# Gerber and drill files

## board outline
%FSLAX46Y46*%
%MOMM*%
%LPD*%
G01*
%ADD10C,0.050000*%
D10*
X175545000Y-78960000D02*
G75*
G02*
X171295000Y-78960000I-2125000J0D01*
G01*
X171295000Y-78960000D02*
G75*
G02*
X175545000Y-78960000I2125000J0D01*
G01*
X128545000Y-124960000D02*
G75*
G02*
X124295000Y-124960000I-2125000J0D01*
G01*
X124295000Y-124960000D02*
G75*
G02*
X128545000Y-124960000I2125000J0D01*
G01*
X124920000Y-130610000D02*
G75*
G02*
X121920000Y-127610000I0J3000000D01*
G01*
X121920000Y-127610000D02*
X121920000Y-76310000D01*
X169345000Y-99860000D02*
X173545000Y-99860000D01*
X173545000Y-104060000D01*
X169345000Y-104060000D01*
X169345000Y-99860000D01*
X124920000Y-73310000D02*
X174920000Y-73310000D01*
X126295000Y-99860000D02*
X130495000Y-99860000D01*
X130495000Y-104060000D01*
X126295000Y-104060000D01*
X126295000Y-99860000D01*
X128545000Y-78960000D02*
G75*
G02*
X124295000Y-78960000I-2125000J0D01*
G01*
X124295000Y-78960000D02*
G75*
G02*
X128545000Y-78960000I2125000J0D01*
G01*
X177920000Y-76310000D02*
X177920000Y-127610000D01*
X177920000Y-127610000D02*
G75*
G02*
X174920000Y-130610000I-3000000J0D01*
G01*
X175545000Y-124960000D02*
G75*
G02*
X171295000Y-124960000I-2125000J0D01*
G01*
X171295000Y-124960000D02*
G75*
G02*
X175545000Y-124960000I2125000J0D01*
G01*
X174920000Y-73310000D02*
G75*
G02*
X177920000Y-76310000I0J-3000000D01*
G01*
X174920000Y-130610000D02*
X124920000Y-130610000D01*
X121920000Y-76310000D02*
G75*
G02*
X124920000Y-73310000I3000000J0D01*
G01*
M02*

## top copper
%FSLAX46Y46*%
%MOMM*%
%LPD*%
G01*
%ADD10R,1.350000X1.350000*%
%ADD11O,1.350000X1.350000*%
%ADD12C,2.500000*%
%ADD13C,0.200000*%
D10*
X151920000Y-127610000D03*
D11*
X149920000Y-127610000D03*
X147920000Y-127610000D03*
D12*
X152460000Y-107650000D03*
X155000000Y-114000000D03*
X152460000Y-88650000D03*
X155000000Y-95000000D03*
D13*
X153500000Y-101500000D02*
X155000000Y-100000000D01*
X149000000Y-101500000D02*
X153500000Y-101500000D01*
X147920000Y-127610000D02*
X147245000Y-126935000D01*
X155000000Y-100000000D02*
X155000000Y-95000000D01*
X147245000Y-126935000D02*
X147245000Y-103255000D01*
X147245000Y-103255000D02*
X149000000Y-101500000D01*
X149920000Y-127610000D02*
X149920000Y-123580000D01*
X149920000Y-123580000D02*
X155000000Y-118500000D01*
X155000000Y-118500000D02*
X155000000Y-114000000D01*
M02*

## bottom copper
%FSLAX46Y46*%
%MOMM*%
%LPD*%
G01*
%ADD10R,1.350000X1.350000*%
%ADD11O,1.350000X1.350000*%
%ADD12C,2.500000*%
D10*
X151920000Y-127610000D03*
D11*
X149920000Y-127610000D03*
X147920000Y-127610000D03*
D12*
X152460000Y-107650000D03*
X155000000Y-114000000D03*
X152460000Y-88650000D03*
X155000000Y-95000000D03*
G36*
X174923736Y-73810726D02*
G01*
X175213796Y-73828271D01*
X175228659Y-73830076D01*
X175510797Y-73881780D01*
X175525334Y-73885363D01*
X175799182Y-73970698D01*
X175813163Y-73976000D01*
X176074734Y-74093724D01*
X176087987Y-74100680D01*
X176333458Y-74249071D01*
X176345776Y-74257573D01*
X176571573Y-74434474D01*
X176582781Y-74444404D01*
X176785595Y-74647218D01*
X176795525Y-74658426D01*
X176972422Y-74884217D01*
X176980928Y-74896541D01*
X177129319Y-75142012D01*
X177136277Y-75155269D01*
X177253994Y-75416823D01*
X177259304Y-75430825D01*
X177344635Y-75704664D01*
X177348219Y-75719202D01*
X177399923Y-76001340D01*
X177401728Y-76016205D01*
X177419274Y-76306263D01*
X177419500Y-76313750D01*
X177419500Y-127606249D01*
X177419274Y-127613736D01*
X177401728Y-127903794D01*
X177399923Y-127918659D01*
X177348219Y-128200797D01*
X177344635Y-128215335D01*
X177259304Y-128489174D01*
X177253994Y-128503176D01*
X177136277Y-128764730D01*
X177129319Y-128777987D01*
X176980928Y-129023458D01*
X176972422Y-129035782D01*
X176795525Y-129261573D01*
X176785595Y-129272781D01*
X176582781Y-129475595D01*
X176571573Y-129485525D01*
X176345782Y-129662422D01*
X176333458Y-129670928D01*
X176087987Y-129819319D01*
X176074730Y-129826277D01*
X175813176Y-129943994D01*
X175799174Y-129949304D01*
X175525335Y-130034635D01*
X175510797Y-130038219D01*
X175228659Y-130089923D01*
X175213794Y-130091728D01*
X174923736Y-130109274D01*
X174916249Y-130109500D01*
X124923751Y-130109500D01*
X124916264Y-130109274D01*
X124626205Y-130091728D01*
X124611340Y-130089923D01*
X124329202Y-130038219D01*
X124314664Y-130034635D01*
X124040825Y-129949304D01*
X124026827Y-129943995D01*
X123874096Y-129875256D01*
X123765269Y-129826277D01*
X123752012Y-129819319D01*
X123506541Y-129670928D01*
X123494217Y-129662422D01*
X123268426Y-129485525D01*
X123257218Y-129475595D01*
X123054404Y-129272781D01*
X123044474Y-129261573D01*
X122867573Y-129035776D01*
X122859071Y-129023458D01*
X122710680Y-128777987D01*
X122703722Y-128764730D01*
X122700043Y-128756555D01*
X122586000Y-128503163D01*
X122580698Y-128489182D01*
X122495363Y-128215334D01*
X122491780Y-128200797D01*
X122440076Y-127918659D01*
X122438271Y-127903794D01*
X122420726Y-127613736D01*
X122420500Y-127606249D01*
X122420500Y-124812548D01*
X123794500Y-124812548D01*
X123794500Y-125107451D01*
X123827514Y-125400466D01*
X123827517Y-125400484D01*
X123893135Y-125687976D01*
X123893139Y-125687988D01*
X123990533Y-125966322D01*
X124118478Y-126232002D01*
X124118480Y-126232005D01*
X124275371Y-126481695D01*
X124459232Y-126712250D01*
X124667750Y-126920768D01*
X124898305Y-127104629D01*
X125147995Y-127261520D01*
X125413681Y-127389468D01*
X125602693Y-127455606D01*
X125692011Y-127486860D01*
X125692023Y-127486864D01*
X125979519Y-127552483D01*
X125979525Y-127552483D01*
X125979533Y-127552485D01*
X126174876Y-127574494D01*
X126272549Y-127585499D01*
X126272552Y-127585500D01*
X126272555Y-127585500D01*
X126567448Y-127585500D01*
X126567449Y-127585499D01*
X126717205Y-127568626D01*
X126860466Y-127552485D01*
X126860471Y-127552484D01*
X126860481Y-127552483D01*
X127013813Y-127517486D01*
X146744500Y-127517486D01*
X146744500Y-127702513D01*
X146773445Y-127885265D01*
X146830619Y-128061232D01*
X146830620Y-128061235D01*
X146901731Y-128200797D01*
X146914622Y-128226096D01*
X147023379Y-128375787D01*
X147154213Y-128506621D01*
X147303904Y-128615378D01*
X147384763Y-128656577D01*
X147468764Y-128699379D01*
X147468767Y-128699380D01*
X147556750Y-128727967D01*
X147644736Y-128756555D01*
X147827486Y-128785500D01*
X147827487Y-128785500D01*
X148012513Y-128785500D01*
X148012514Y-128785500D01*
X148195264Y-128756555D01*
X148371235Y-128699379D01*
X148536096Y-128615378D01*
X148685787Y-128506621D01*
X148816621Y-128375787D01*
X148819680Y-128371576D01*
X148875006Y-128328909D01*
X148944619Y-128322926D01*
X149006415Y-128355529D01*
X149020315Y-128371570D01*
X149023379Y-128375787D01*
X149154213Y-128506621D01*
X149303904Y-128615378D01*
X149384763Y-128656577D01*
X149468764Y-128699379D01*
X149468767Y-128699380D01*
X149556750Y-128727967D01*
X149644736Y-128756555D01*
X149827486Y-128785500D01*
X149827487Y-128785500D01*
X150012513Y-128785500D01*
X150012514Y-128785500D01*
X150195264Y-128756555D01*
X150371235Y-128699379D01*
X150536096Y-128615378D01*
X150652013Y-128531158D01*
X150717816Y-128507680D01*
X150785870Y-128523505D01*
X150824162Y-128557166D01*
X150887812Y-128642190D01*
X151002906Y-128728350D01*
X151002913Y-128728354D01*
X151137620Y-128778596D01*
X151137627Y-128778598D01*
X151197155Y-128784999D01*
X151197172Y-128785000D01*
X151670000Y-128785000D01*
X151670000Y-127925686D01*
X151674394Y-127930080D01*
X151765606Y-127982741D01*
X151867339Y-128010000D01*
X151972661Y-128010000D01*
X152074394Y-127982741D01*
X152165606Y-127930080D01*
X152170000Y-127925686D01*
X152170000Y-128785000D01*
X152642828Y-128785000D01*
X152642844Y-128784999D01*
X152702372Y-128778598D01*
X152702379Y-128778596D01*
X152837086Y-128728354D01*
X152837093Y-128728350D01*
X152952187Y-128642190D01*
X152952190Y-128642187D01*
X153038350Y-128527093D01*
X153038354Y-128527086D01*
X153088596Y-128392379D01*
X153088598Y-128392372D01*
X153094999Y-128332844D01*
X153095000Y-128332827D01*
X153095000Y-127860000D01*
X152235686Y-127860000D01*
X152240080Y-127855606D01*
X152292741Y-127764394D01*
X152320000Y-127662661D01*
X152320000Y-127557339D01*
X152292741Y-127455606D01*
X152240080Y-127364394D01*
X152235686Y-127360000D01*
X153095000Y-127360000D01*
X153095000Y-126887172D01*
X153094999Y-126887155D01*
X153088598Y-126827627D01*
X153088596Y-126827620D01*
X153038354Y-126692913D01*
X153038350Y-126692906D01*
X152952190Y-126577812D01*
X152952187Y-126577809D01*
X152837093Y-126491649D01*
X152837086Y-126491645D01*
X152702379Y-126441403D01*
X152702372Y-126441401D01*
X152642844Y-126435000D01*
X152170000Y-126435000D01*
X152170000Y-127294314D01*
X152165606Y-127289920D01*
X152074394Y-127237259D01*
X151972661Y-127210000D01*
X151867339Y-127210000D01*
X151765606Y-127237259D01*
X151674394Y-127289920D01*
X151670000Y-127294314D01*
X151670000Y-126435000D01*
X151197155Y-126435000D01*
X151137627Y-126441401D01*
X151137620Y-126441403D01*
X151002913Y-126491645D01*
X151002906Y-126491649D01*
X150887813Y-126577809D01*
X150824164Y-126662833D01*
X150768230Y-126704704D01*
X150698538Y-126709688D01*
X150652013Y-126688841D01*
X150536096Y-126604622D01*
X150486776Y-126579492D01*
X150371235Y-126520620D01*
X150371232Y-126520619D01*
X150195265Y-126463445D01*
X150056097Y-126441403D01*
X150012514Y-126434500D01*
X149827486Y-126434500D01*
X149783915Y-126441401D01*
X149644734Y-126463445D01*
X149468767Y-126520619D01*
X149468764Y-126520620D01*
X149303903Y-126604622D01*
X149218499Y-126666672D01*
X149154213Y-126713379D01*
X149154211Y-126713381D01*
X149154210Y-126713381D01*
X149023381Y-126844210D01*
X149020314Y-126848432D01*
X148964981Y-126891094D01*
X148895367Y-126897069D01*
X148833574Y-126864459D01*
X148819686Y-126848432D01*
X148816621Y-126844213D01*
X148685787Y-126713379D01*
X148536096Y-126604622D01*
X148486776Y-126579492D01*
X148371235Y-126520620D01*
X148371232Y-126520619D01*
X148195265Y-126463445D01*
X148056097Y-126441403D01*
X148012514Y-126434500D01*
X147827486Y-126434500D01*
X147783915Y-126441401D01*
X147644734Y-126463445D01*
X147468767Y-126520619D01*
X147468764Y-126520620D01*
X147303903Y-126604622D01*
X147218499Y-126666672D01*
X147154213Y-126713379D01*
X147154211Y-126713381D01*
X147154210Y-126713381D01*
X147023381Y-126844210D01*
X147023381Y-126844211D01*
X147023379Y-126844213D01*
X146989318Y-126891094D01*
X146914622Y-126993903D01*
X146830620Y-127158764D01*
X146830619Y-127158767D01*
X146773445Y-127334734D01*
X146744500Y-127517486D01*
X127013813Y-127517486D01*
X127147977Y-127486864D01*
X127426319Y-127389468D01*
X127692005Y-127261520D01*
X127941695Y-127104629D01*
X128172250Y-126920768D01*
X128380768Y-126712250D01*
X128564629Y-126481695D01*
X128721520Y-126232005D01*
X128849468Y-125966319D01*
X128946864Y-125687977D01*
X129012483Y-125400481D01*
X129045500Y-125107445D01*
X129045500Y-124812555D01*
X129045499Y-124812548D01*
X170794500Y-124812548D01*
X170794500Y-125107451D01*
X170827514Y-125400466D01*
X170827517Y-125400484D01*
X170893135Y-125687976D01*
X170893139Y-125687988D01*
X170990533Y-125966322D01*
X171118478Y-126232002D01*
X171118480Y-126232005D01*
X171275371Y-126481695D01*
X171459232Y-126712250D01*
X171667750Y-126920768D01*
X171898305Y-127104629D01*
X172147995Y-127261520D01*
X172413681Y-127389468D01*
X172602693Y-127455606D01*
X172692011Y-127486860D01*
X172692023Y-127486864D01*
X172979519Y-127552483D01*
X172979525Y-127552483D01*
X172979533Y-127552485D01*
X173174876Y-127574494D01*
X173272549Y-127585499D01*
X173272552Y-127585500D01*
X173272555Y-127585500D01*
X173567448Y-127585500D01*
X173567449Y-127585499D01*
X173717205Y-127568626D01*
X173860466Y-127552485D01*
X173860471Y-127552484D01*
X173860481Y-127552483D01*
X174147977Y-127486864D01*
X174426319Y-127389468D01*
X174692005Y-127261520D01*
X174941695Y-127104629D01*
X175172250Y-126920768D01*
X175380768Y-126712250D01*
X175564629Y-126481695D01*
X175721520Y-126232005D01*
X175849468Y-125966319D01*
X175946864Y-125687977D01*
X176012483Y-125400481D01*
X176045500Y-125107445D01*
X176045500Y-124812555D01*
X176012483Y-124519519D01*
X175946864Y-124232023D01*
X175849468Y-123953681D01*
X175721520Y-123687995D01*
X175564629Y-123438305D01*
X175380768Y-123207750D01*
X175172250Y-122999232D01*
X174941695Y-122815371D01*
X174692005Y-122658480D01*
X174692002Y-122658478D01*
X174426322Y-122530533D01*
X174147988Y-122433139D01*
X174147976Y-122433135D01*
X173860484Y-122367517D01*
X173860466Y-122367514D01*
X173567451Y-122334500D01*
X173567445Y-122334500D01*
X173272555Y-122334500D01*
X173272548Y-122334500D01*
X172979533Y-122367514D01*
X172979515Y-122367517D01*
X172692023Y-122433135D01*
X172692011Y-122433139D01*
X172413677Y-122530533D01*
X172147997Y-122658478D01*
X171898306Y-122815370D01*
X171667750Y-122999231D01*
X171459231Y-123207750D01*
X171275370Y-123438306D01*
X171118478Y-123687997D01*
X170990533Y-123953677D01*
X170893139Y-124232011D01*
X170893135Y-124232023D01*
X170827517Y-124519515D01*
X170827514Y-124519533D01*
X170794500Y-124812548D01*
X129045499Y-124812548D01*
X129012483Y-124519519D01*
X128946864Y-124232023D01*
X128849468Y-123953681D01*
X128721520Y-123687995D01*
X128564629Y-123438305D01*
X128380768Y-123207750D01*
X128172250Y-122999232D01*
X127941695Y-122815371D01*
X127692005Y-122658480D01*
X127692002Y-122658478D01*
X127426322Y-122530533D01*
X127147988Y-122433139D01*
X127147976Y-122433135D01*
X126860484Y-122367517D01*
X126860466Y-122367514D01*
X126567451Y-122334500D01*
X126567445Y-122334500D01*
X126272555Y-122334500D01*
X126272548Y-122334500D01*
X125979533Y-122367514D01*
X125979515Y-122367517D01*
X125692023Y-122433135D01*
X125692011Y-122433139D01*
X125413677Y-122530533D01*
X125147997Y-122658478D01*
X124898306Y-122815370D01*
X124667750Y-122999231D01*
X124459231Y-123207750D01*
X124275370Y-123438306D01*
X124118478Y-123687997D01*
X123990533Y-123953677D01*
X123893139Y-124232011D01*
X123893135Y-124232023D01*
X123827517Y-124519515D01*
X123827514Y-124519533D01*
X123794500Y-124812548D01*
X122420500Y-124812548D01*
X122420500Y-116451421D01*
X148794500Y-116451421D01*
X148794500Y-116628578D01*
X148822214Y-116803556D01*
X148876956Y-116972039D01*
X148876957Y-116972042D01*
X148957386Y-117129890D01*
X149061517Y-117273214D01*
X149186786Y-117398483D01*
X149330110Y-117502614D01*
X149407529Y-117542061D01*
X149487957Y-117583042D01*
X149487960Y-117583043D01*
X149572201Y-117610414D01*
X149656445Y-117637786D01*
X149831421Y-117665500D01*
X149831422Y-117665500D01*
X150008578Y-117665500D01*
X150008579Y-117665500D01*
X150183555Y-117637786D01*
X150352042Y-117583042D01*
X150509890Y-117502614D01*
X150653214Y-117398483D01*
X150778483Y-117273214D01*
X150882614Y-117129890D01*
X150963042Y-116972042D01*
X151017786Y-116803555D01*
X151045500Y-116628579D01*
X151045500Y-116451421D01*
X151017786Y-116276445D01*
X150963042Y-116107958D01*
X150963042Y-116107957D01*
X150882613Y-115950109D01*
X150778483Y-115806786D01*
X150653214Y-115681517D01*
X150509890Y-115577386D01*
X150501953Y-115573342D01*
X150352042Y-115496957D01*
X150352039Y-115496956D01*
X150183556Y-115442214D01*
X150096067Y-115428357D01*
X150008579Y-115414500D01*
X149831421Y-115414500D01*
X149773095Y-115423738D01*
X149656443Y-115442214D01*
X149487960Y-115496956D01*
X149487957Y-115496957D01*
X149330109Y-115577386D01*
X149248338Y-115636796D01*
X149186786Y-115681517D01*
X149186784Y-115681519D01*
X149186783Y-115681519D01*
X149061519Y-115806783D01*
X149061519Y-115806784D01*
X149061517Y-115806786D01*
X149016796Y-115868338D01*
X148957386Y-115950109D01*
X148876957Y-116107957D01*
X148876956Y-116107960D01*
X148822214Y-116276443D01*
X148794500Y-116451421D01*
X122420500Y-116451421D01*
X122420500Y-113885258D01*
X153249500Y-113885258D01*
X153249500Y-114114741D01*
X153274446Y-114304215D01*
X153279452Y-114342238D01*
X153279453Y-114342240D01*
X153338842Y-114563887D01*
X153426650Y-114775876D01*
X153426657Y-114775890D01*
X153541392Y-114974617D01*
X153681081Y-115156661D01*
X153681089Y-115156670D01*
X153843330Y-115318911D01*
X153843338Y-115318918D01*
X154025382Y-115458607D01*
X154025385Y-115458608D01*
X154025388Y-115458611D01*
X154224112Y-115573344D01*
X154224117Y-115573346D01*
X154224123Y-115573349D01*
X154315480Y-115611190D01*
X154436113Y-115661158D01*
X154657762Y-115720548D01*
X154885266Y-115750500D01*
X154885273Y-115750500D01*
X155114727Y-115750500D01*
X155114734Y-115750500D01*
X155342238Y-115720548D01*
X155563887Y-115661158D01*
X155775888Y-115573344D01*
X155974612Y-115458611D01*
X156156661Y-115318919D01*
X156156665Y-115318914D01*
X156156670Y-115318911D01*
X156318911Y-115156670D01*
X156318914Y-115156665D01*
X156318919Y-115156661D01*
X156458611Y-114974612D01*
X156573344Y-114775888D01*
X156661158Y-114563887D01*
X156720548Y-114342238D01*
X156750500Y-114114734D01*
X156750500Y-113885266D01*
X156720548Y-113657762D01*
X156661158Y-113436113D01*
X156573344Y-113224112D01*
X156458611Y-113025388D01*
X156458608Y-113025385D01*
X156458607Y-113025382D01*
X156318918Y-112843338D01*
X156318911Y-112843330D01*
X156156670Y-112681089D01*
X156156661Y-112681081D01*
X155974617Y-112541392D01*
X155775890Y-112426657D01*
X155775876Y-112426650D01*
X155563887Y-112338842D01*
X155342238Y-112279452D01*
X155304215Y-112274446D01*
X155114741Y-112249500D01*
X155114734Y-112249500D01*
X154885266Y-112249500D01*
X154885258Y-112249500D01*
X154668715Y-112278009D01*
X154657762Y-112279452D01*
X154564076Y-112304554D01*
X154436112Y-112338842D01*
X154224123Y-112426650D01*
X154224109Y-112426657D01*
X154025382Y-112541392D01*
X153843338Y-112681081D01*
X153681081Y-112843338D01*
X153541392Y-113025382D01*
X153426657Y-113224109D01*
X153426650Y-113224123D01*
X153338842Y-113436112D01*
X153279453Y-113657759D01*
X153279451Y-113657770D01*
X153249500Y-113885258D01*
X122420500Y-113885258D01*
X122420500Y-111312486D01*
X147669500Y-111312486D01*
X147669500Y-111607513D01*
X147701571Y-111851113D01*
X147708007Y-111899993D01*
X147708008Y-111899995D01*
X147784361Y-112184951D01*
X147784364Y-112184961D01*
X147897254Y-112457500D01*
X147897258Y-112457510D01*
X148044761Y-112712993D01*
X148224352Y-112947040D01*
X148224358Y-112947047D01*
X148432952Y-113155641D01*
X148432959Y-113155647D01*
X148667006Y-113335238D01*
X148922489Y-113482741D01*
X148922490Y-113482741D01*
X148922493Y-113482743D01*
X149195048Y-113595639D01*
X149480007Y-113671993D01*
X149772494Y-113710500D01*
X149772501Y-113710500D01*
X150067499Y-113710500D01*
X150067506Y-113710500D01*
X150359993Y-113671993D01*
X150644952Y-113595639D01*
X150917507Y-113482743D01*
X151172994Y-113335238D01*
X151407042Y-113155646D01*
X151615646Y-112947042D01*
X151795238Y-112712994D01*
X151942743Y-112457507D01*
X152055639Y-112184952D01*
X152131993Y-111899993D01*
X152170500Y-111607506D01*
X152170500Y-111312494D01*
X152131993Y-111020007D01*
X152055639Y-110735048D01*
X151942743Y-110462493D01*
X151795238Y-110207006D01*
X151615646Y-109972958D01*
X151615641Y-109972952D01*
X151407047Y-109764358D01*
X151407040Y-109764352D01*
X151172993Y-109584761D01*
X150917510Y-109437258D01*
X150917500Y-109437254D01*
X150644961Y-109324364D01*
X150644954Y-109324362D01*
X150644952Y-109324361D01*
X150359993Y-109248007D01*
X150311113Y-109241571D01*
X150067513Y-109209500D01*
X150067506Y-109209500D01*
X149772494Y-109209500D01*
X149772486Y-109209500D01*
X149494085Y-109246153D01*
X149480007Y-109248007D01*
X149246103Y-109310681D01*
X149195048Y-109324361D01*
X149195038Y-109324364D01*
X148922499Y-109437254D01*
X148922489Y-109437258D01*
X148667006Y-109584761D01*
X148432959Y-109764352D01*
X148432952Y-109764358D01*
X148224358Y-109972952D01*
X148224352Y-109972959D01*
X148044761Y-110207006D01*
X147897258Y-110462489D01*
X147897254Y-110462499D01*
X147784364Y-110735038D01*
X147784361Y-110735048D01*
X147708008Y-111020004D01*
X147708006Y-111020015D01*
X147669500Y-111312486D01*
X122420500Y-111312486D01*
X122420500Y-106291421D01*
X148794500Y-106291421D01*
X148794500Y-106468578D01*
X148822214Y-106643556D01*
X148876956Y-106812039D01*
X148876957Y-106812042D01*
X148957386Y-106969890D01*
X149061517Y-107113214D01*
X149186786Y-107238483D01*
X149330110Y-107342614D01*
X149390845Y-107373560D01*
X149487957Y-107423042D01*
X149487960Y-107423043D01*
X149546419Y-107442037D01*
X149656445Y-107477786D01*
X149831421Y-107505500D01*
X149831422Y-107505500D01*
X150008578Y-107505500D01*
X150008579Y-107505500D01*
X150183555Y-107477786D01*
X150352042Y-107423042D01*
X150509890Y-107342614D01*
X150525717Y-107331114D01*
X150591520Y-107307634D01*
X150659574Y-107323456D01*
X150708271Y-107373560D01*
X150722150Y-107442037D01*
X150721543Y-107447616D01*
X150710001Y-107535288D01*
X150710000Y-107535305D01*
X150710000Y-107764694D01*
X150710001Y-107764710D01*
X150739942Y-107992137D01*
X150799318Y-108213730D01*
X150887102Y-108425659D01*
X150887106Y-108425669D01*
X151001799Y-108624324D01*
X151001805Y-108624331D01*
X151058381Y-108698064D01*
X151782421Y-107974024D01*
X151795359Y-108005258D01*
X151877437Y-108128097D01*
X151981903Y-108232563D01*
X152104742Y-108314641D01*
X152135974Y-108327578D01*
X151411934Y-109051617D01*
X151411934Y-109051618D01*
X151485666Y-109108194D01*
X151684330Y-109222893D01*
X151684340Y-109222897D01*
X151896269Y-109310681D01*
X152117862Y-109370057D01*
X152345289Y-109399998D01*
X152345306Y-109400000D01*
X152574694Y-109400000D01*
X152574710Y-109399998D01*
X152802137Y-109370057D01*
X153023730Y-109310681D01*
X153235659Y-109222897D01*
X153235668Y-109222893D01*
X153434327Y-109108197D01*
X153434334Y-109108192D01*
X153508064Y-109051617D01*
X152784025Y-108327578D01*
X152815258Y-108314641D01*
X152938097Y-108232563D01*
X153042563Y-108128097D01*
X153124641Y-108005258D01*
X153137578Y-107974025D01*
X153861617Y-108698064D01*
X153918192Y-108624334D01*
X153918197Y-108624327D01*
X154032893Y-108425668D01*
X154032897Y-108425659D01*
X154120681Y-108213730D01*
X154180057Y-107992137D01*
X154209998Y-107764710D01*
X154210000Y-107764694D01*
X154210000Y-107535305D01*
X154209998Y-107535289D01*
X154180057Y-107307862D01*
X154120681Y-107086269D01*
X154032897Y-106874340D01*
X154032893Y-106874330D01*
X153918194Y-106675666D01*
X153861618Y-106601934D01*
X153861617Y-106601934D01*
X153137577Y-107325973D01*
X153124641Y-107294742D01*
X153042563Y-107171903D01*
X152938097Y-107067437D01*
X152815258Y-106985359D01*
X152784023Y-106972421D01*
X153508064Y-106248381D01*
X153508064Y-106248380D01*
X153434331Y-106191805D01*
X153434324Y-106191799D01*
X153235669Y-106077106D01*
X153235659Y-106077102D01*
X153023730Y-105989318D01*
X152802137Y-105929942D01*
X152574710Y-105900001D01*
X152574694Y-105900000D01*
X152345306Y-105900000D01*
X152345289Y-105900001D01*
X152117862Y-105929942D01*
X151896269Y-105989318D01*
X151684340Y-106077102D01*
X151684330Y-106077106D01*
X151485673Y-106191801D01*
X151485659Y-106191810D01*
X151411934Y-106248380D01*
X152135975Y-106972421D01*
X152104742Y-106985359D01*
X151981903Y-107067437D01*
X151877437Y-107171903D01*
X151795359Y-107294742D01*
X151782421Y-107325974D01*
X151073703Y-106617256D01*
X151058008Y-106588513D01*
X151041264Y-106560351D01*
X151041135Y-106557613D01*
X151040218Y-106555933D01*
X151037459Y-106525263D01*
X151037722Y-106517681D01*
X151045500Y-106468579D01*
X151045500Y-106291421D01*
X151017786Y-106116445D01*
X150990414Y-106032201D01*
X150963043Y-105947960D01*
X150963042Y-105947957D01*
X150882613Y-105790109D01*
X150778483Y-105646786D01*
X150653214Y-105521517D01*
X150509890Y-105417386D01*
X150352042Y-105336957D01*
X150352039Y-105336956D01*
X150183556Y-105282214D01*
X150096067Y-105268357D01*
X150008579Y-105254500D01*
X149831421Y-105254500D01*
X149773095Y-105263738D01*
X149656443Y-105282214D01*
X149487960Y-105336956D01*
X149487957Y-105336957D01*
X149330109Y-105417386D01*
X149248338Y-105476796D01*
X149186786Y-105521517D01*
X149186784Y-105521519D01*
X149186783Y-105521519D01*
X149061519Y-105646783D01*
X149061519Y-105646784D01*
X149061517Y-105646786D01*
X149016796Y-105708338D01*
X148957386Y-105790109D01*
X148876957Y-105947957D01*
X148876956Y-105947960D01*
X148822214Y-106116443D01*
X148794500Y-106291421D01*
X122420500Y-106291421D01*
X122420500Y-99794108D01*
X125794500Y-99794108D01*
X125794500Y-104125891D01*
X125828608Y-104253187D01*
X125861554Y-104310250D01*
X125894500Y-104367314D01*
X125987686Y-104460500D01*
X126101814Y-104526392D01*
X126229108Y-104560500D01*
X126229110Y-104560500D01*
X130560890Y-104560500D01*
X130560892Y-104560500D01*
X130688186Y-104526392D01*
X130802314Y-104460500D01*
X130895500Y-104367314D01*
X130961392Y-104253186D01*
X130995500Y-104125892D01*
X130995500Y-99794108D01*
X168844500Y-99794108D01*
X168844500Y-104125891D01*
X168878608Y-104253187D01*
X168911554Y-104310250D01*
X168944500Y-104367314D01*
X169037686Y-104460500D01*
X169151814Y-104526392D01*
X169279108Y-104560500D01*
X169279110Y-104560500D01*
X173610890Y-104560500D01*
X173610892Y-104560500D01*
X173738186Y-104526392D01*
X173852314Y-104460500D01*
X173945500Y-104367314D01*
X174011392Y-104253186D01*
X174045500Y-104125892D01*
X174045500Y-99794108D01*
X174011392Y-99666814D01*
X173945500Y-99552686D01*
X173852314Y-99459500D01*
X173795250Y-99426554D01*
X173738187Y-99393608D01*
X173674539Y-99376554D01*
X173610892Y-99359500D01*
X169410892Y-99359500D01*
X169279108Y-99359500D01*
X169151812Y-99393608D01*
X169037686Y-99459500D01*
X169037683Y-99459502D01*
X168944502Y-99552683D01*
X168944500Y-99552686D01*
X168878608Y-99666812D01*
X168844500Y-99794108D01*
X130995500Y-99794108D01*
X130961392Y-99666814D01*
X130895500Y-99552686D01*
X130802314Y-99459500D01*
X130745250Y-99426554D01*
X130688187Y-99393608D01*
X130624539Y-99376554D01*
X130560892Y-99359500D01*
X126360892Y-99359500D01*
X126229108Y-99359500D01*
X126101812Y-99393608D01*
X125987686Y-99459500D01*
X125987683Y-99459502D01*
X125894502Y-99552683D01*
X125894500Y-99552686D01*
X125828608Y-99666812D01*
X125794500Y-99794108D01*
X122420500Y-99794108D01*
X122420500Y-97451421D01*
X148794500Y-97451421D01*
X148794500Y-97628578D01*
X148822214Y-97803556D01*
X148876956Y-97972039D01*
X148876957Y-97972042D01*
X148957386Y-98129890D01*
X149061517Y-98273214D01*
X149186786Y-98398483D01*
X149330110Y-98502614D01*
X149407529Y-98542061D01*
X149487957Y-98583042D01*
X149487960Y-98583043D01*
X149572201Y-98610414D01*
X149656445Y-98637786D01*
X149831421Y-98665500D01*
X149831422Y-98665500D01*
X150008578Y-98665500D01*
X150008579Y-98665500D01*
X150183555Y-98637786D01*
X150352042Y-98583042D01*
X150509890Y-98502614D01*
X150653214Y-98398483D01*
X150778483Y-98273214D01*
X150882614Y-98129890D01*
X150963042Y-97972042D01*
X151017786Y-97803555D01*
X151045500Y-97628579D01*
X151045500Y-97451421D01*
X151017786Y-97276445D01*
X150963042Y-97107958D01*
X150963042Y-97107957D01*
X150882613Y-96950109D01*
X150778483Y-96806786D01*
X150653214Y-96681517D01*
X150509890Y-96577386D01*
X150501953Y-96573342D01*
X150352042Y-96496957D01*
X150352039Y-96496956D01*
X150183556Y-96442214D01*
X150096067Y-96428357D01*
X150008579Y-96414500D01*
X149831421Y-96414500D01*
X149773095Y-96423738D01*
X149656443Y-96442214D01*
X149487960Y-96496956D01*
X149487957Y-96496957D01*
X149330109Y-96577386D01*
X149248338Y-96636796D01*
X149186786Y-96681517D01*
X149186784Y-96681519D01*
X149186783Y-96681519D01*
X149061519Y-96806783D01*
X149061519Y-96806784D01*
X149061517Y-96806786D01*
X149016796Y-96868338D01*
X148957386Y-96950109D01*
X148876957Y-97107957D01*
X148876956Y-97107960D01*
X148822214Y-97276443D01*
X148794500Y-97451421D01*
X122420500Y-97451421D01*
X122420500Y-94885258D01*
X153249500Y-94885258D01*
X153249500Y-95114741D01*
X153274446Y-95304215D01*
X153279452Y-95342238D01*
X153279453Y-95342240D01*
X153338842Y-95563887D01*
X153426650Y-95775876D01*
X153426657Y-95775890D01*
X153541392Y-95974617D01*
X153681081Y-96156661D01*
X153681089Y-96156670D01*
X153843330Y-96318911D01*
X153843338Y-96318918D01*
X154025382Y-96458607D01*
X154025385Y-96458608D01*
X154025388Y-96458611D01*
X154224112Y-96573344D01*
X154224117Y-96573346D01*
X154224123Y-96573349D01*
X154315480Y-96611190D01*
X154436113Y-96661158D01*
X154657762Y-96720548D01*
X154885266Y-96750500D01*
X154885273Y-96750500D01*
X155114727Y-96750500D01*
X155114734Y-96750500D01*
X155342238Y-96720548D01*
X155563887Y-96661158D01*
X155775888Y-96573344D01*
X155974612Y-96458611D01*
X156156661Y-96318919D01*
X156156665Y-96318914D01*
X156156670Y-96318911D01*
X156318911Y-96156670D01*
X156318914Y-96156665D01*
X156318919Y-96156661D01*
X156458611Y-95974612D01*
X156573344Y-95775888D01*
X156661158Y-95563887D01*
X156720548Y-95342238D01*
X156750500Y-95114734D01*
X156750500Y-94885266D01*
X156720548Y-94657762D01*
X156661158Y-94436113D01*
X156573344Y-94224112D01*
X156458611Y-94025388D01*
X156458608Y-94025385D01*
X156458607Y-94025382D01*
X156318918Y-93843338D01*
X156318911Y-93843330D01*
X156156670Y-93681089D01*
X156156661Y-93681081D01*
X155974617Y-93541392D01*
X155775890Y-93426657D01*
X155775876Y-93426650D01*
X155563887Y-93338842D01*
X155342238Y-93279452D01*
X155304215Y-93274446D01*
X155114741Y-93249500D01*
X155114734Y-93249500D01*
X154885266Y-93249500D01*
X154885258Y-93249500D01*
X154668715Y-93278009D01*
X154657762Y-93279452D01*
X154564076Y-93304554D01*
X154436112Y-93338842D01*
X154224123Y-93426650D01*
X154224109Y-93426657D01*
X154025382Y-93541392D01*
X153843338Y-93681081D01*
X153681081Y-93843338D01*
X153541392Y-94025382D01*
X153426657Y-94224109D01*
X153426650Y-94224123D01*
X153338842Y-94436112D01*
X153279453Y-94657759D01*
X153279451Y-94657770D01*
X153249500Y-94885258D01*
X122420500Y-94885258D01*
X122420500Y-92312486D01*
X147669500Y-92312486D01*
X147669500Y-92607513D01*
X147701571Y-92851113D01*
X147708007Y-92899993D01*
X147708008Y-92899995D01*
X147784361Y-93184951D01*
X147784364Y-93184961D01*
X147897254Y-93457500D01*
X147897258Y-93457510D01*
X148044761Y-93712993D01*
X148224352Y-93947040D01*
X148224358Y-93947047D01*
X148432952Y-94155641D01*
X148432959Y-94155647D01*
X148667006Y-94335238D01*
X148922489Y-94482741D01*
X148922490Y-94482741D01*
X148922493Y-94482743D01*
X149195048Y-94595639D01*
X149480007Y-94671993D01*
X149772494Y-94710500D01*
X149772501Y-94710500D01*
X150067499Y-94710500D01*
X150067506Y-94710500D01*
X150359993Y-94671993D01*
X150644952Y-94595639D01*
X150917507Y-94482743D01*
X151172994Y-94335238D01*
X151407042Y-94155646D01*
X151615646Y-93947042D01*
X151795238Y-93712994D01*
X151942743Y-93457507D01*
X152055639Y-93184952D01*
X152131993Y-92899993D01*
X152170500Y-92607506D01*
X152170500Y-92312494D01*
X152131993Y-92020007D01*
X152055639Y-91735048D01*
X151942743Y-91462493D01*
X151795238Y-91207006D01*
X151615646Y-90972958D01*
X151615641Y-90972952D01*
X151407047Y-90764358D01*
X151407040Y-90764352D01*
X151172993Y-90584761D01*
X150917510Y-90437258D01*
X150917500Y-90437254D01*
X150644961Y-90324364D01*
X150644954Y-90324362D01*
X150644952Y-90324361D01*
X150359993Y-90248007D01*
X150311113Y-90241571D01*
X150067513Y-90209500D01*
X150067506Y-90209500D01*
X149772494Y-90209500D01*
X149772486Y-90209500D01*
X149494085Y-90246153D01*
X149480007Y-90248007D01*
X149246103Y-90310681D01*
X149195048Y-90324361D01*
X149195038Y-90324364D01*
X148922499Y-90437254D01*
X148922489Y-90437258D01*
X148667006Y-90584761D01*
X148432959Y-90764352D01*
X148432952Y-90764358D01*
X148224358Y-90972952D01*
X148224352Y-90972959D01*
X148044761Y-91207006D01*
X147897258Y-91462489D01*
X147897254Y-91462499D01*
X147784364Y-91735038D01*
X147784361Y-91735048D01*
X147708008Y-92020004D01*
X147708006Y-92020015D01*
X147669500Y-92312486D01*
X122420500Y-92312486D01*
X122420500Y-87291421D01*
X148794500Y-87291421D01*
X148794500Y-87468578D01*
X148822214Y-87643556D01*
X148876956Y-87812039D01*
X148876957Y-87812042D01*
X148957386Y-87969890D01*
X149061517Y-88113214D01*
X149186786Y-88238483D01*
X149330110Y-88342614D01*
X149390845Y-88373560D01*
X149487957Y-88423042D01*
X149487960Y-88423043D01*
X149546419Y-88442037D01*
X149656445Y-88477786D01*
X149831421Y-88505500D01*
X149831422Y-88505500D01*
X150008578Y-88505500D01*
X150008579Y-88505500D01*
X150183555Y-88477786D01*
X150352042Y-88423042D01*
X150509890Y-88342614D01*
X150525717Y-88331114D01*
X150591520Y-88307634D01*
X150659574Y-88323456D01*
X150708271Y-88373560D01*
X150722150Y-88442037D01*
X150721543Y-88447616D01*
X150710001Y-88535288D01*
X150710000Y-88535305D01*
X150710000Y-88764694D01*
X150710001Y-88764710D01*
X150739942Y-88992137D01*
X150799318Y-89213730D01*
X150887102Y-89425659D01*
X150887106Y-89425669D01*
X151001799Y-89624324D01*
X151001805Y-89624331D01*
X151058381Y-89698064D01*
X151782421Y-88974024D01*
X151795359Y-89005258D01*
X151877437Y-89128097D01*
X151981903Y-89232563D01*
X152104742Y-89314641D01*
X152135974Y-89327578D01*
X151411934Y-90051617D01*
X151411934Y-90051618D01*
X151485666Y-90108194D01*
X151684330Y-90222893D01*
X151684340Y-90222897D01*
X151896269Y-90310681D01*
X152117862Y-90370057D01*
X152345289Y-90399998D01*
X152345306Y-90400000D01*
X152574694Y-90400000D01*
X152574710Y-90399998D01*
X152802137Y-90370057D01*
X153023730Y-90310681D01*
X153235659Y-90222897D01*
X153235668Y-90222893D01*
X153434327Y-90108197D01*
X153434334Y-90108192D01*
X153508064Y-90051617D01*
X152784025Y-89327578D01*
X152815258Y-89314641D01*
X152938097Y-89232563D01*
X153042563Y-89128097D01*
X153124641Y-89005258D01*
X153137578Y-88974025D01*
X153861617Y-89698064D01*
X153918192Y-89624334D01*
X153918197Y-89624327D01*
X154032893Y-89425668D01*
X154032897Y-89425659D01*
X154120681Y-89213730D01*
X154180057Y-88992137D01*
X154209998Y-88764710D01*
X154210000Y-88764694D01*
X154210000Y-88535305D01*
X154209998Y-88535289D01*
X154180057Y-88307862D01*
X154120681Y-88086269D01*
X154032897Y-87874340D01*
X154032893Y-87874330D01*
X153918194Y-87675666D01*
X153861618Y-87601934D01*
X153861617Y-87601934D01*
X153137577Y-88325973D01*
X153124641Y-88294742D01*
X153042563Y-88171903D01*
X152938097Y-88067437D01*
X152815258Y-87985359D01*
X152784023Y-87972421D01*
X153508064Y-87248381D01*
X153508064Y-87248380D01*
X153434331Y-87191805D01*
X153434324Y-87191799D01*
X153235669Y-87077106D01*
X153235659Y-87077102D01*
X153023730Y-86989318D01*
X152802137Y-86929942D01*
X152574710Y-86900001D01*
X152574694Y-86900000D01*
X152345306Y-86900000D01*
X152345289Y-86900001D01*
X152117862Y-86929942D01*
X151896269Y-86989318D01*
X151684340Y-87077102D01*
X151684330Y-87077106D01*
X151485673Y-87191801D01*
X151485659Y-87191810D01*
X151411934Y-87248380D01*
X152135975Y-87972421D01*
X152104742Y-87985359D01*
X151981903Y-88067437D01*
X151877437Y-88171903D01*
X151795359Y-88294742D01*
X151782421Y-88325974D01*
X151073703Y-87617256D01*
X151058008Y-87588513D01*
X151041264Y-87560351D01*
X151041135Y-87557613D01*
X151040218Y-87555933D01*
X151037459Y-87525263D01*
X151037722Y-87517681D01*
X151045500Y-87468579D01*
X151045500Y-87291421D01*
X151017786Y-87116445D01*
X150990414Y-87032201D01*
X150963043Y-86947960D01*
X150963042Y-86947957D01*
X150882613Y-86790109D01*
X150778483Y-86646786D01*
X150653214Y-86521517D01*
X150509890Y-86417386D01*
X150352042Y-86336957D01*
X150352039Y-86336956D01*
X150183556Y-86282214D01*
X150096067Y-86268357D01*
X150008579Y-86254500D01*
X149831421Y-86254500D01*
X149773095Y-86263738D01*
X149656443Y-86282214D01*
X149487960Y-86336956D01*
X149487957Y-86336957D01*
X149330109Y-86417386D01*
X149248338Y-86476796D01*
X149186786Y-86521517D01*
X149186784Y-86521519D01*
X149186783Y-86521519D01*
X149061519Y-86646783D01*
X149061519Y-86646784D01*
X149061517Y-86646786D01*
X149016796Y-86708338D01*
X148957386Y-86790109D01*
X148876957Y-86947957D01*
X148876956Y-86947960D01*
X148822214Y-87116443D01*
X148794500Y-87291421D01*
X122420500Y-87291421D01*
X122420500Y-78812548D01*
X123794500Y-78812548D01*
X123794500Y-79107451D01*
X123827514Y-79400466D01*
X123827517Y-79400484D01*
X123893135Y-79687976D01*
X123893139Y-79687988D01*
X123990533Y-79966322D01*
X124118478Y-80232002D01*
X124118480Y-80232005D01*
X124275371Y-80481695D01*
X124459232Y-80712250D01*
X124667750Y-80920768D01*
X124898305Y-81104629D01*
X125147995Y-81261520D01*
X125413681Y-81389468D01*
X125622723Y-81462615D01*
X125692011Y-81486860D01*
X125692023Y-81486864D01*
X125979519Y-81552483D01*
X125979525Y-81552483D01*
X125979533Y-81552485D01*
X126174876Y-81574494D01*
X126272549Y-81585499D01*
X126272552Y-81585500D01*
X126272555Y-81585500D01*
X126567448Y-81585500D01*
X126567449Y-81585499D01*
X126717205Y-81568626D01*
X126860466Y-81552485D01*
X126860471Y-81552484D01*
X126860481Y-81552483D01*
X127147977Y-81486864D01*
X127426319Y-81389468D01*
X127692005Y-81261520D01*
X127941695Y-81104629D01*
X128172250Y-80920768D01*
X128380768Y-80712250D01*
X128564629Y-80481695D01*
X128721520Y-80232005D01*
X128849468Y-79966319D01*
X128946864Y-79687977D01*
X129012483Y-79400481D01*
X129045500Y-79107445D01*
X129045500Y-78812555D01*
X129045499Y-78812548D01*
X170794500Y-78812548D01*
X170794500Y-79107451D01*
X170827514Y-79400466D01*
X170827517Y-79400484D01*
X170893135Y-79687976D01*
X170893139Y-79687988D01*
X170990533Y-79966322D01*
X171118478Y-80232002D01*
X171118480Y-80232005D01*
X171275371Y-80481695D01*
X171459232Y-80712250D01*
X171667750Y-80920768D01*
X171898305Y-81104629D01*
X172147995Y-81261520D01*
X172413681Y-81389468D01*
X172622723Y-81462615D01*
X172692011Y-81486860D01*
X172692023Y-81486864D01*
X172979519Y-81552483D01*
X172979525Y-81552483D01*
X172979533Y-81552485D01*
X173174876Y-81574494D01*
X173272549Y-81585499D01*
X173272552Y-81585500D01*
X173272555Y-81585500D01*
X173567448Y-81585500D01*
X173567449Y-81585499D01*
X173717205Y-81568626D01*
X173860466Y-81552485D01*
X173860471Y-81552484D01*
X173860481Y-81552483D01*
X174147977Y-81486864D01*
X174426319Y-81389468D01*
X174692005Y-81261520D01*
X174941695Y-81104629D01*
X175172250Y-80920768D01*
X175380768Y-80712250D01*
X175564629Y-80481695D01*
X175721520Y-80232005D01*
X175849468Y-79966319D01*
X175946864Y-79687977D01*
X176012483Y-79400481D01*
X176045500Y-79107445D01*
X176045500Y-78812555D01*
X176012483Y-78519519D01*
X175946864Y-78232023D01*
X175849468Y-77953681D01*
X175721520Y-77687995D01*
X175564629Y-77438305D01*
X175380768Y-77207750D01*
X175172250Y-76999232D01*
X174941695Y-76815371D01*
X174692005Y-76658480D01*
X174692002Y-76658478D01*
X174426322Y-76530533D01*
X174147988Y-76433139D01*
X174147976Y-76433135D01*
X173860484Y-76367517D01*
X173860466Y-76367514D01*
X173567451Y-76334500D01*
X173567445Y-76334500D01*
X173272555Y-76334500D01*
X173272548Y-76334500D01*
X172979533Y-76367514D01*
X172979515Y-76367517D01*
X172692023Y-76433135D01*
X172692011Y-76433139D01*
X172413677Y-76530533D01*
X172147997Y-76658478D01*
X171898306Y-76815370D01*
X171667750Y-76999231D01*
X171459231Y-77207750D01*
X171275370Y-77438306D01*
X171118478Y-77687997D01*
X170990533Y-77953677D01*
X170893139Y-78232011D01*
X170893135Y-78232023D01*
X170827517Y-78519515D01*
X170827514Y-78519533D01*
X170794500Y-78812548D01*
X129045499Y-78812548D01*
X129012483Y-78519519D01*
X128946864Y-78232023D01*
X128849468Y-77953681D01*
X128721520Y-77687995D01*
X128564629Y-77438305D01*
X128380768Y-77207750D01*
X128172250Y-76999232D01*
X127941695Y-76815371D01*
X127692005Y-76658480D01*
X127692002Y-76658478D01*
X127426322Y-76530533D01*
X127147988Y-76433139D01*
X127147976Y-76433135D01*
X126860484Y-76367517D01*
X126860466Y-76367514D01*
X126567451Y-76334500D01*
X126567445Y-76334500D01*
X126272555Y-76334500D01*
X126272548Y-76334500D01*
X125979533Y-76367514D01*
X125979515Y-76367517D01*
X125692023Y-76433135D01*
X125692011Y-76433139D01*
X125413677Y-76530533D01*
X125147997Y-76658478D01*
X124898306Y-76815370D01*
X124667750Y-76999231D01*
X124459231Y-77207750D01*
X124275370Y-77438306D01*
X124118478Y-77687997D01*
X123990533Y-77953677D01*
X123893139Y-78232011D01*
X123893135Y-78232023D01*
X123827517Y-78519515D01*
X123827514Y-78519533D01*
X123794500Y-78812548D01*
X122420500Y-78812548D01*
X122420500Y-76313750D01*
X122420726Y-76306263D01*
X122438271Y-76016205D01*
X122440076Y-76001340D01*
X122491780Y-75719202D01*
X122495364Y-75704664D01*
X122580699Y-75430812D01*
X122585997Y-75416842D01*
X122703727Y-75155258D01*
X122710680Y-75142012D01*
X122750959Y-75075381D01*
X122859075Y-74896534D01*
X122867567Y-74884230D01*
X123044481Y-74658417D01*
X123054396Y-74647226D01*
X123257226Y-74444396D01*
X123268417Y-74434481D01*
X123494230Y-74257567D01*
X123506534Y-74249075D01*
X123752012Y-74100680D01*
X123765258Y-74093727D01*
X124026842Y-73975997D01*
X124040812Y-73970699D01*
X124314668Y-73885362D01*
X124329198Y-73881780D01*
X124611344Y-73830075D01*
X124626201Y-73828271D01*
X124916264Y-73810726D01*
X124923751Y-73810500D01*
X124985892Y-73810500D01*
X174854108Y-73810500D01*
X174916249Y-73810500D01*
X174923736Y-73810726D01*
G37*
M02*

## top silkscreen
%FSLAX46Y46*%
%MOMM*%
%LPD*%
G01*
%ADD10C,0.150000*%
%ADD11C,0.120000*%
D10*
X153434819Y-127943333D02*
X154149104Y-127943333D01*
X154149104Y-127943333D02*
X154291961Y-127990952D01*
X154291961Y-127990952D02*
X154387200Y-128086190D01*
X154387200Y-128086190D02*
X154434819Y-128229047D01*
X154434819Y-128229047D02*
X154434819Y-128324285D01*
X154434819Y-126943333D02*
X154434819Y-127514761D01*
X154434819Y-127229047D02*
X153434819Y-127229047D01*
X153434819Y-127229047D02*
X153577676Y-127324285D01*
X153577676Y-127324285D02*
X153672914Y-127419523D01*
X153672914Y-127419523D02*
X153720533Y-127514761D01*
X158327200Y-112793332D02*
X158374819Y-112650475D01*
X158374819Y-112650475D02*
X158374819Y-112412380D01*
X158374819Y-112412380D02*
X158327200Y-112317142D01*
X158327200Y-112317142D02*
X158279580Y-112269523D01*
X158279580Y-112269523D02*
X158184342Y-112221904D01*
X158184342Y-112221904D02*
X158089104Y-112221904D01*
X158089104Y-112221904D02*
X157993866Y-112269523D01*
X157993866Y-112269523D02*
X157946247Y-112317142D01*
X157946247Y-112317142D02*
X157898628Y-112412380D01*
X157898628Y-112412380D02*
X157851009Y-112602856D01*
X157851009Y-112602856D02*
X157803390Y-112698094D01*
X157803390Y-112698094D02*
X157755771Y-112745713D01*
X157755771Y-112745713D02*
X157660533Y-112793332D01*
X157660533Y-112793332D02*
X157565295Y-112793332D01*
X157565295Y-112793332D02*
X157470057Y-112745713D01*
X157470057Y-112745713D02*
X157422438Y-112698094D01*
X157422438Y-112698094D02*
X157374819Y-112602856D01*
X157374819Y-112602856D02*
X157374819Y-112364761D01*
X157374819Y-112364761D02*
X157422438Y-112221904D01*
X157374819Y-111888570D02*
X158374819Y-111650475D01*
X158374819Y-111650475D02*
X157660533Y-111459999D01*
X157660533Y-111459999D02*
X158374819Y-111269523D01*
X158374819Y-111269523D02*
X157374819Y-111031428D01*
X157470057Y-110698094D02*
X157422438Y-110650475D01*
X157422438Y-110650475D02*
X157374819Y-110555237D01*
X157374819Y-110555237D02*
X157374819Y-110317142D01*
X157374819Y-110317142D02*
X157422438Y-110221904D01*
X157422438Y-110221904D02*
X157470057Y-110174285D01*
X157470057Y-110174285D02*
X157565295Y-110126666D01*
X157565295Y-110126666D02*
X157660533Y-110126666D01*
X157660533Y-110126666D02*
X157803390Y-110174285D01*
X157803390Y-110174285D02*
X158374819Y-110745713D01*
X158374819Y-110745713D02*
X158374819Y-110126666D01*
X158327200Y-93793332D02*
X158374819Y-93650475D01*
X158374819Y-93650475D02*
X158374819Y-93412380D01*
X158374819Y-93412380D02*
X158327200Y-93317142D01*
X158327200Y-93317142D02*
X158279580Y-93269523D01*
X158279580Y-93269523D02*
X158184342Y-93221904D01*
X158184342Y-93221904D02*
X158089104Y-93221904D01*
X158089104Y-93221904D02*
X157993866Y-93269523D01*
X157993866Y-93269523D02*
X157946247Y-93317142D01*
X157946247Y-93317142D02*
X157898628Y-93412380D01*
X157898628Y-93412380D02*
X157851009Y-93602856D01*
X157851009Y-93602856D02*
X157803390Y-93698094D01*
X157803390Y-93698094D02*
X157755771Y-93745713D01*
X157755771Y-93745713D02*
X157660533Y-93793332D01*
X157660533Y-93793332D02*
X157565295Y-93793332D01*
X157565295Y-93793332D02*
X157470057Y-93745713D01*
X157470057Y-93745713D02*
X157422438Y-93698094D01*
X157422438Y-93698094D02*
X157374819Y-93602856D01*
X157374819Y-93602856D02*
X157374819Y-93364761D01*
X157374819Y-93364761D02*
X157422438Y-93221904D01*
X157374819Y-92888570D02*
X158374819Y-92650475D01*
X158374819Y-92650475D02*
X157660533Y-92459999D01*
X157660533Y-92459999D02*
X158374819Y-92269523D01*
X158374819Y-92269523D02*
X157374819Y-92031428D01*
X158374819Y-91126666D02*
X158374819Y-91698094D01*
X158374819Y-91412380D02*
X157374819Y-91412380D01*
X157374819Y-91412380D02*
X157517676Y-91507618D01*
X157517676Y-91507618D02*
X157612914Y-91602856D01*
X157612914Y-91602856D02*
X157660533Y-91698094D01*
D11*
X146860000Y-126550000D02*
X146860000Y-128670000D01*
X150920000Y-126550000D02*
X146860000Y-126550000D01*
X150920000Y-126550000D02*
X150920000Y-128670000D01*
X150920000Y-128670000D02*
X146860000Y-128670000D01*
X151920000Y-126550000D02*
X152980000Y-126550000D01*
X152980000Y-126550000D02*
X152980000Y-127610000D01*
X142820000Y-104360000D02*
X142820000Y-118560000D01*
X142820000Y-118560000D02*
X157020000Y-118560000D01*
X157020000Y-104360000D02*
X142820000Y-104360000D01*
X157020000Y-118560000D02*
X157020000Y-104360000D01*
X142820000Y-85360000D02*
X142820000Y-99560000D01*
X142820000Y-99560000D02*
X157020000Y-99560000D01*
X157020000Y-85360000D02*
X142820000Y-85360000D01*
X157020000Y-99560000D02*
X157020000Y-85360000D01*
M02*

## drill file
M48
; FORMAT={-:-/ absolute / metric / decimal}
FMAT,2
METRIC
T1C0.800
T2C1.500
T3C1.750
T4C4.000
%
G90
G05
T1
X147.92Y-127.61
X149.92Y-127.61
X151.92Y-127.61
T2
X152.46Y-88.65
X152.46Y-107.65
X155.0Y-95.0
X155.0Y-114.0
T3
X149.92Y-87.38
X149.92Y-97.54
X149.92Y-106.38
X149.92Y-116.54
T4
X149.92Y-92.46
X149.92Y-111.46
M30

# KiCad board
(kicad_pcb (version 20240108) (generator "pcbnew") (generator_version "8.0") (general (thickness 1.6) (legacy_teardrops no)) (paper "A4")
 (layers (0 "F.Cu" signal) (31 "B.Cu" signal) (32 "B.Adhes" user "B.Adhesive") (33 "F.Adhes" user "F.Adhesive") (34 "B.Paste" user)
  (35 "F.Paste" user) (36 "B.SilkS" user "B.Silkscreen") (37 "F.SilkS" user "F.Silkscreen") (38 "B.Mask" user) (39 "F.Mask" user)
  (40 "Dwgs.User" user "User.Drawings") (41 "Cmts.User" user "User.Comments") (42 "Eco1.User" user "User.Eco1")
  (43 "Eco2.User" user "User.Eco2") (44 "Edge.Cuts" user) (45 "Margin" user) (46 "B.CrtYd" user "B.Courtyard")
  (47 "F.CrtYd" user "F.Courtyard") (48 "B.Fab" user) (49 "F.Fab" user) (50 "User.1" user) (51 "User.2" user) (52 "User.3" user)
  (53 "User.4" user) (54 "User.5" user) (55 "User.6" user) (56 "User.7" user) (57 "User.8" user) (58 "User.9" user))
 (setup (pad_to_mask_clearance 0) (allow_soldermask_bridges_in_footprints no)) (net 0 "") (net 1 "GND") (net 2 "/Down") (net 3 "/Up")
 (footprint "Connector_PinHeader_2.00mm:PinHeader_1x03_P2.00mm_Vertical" (layer "F.Cu") (at 151.92 127.61 -90)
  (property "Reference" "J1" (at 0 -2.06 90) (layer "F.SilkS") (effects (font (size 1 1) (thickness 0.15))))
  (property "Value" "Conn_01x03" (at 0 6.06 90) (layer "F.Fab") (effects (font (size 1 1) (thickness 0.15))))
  (fp_line (start -1.06 5.06) (end 1.06 5.06) (stroke (width 0.12) (type solid)) (layer "F.SilkS"))
  (fp_line (start -1.06 1) (end -1.06 5.06) (stroke (width 0.12) (type solid)) (layer "F.SilkS"))
  (fp_line (start -1.06 1) (end 1.06 1) (stroke (width 0.12) (type solid)) (layer "F.SilkS"))
  (fp_line (start 1.06 1) (end 1.06 5.06) (stroke (width 0.12) (type solid)) (layer "F.SilkS"))
  (fp_line (start -1.06 0) (end -1.06 -1.06) (stroke (width 0.12) (type solid)) (layer "F.SilkS"))
  (fp_line (start -1.06 -1.06) (end 0 -1.06) (stroke (width 0.12) (type solid)) (layer "F.SilkS"))
  (pad "1" thru_hole rect (at 0 0 270) (size 1.35 1.35) (drill 0.8) (layers "*.Cu" "*.Mask") (remove_unused_layers no) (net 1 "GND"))
  (pad "2" thru_hole oval (at 0 2 270) (size 1.35 1.35) (drill 0.8) (layers "*.Cu" "*.Mask") (remove_unused_layers no) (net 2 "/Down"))
  (pad "3" thru_hole oval (at 0 4 270) (size 1.35 1.35) (drill 0.8) (layers "*.Cu" "*.Mask") (remove_unused_layers no) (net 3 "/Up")))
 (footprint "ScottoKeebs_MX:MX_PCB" (layer "F.Cu") (at 149.92 111.46 -90)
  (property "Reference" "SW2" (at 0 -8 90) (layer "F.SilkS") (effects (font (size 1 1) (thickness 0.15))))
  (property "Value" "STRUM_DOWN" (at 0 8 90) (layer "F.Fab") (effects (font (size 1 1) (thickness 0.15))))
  (fp_line (start -7.1 7.1) (end 7.1 7.1) (stroke (width 0.12) (type solid)) (layer "F.SilkS"))
  (fp_line (start 7.1 7.1) (end 7.1 -7.1) (stroke (width 0.12) (type solid)) (layer "F.SilkS"))
  (fp_line (start -7.1 -7.1) (end -7.1 7.1) (stroke (width 0.12) (type solid)) (layer "F.SilkS"))
  (fp_line (start 7.1 -7.1) (end -7.1 -7.1) (stroke (width 0.12) (type solid)) (layer "F.SilkS"))
  (pad "" np_thru_hole circle (at -5.08 0 270) (size 1.75 1.75) (drill 1.75) (layers "*.Cu" "*.Mask"))
  (pad "" np_thru_hole circle (at 0 0 270) (size 4 4) (drill 4) (layers "*.Cu" "*.Mask"))
  (pad "" np_thru_hole circle (at 5.08 0 270) (size 1.75 1.75) (drill 1.75) (layers "*.Cu" "*.Mask"))
  (pad "1" thru_hole circle (at -3.81 -2.54 270) (size 2.5 2.5) (drill 1.5) (layers "*.Cu" "*.Mask") (remove_unused_layers no) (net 1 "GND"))
  (pad "2" thru_hole circle (at 2.54 -5.08 270) (size 2.5 2.5) (drill 1.5) (layers "*.Cu" "*.Mask") (remove_unused_layers no)
   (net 2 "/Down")))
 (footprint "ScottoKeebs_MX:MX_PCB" (layer "F.Cu") (at 149.92 92.46 -90)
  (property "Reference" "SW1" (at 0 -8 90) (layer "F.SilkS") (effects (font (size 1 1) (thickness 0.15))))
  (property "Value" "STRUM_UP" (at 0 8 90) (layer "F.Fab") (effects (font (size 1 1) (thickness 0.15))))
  (fp_line (start -7.1 7.1) (end 7.1 7.1) (stroke (width 0.12) (type solid)) (layer "F.SilkS"))
  (fp_line (start 7.1 7.1) (end 7.1 -7.1) (stroke (width 0.12) (type solid)) (layer "F.SilkS"))
  (fp_line (start -7.1 -7.1) (end -7.1 7.1) (stroke (width 0.12) (type solid)) (layer "F.SilkS"))
  (fp_line (start 7.1 -7.1) (end -7.1 -7.1) (stroke (width 0.12) (type solid)) (layer "F.SilkS"))
  (pad "" np_thru_hole circle (at -5.08 0 270) (size 1.75 1.75) (drill 1.75) (layers "*.Cu" "*.Mask"))
  (pad "" np_thru_hole circle (at 0 0 270) (size 4 4) (drill 4) (layers "*.Cu" "*.Mask"))
  (pad "" np_thru_hole circle (at 5.08 0 270) (size 1.75 1.75) (drill 1.75) (layers "*.Cu" "*.Mask"))
  (pad "1" thru_hole circle (at -3.81 -2.54 270) (size 2.5 2.5) (drill 1.5) (layers "*.Cu" "*.Mask") (remove_unused_layers no) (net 1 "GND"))
  (pad "2" thru_hole circle (at 2.54 -5.08 270) (size 2.5 2.5) (drill 1.5) (layers "*.Cu" "*.Mask") (remove_unused_layers no) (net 3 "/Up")))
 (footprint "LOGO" (layer "B.Cu") (at 135.636 89.662 180)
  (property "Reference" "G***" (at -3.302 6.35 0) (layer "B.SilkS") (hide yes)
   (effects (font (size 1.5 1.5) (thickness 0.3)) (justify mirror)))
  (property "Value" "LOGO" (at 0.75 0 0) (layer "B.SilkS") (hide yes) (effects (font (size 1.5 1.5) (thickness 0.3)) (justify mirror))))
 (gr_circle (center 173.42 78.96) (end 175.545 78.96) (stroke (width 0.05) (type default)) (fill none) (layer "Edge.Cuts"))
 (gr_circle (center 126.42 124.96) (end 128.545 124.96) (stroke (width 0.05) (type default)) (fill none) (layer "Edge.Cuts"))
 (gr_arc (start 124.92 130.61) (mid 122.79868 129.73132) (end 121.92 127.61) (stroke (width 0.05) (type default)) (layer "Edge.Cuts"))
 (gr_line (start 121.92 127.61) (end 121.92 76.31) (stroke (width 0.05) (type default)) (layer "Edge.Cuts"))
 (gr_rect (start 169.345 99.86) (end 173.545 104.06) (stroke (width 0.05) (type default)) (fill none) (layer "Edge.Cuts"))
 (gr_line (start 124.92 73.31) (end 174.92 73.31) (stroke (width 0.05) (type default)) (layer "Edge.Cuts"))
 (gr_rect (start 126.295 99.86) (end 130.495 104.06) (stroke (width 0.05) (type default)) (fill none) (layer "Edge.Cuts"))
 (gr_circle (center 126.42 78.96) (end 128.545 78.96) (stroke (width 0.05) (type default)) (fill none) (layer "Edge.Cuts"))
 (gr_line (start 177.92 76.31) (end 177.92 127.61) (stroke (width 0.05) (type default)) (layer "Edge.Cuts"))
 (gr_arc (start 177.92 127.61) (mid 177.04132 129.73132) (end 174.92 130.61) (stroke (width 0.05) (type default)) (layer "Edge.Cuts"))
 (gr_circle (center 173.42 124.96) (end 175.545 124.96) (stroke (width 0.05) (type default)) (fill none) (layer "Edge.Cuts"))
 (gr_arc (start 174.92 73.31) (mid 177.04132 74.18868) (end 177.92 76.31) (stroke (width 0.05) (type default)) (layer "Edge.Cuts"))
 (gr_line (start 174.92 130.61) (end 124.92 130.61) (stroke (width 0.05) (type default)) (layer "Edge.Cuts"))
 (gr_arc (start 121.92 76.31) (mid 122.79868 74.18868) (end 124.92 73.31) (stroke (width 0.05) (type default)) (layer "Edge.Cuts"))
 (segment (start 153.5 101.5) (end 155 100) (width 0.2) (layer "F.Cu") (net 3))
 (segment (start 149 101.5) (end 153.5 101.5) (width 0.2) (layer "F.Cu") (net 3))
 (segment (start 147.92 127.61) (end 147.245 126.935) (width 0.2) (layer "F.Cu") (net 3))
 (segment (start 155 100) (end 155 95) (width 0.2) (layer "F.Cu") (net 3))
 (segment (start 147.245 126.935) (end 147.245 103.255) (width 0.2) (layer "F.Cu") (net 3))
 (segment (start 147.245 103.255) (end 149 101.5) (width 0.2) (layer "F.Cu") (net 3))
 (segment (start 149.92 127.61) (end 149.92 123.58) (width 0.2) (layer "F.Cu") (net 2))
 (segment (start 149.92 123.58) (end 155 118.5) (width 0.2) (layer "F.Cu") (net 2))
 (segment (start 155 118.5) (end 155 114) (width 0.2) (layer "F.Cu") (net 2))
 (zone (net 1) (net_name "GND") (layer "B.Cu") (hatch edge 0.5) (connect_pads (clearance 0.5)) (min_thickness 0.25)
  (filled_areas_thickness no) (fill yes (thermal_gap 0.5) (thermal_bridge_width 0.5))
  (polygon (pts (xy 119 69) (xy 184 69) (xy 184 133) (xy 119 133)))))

